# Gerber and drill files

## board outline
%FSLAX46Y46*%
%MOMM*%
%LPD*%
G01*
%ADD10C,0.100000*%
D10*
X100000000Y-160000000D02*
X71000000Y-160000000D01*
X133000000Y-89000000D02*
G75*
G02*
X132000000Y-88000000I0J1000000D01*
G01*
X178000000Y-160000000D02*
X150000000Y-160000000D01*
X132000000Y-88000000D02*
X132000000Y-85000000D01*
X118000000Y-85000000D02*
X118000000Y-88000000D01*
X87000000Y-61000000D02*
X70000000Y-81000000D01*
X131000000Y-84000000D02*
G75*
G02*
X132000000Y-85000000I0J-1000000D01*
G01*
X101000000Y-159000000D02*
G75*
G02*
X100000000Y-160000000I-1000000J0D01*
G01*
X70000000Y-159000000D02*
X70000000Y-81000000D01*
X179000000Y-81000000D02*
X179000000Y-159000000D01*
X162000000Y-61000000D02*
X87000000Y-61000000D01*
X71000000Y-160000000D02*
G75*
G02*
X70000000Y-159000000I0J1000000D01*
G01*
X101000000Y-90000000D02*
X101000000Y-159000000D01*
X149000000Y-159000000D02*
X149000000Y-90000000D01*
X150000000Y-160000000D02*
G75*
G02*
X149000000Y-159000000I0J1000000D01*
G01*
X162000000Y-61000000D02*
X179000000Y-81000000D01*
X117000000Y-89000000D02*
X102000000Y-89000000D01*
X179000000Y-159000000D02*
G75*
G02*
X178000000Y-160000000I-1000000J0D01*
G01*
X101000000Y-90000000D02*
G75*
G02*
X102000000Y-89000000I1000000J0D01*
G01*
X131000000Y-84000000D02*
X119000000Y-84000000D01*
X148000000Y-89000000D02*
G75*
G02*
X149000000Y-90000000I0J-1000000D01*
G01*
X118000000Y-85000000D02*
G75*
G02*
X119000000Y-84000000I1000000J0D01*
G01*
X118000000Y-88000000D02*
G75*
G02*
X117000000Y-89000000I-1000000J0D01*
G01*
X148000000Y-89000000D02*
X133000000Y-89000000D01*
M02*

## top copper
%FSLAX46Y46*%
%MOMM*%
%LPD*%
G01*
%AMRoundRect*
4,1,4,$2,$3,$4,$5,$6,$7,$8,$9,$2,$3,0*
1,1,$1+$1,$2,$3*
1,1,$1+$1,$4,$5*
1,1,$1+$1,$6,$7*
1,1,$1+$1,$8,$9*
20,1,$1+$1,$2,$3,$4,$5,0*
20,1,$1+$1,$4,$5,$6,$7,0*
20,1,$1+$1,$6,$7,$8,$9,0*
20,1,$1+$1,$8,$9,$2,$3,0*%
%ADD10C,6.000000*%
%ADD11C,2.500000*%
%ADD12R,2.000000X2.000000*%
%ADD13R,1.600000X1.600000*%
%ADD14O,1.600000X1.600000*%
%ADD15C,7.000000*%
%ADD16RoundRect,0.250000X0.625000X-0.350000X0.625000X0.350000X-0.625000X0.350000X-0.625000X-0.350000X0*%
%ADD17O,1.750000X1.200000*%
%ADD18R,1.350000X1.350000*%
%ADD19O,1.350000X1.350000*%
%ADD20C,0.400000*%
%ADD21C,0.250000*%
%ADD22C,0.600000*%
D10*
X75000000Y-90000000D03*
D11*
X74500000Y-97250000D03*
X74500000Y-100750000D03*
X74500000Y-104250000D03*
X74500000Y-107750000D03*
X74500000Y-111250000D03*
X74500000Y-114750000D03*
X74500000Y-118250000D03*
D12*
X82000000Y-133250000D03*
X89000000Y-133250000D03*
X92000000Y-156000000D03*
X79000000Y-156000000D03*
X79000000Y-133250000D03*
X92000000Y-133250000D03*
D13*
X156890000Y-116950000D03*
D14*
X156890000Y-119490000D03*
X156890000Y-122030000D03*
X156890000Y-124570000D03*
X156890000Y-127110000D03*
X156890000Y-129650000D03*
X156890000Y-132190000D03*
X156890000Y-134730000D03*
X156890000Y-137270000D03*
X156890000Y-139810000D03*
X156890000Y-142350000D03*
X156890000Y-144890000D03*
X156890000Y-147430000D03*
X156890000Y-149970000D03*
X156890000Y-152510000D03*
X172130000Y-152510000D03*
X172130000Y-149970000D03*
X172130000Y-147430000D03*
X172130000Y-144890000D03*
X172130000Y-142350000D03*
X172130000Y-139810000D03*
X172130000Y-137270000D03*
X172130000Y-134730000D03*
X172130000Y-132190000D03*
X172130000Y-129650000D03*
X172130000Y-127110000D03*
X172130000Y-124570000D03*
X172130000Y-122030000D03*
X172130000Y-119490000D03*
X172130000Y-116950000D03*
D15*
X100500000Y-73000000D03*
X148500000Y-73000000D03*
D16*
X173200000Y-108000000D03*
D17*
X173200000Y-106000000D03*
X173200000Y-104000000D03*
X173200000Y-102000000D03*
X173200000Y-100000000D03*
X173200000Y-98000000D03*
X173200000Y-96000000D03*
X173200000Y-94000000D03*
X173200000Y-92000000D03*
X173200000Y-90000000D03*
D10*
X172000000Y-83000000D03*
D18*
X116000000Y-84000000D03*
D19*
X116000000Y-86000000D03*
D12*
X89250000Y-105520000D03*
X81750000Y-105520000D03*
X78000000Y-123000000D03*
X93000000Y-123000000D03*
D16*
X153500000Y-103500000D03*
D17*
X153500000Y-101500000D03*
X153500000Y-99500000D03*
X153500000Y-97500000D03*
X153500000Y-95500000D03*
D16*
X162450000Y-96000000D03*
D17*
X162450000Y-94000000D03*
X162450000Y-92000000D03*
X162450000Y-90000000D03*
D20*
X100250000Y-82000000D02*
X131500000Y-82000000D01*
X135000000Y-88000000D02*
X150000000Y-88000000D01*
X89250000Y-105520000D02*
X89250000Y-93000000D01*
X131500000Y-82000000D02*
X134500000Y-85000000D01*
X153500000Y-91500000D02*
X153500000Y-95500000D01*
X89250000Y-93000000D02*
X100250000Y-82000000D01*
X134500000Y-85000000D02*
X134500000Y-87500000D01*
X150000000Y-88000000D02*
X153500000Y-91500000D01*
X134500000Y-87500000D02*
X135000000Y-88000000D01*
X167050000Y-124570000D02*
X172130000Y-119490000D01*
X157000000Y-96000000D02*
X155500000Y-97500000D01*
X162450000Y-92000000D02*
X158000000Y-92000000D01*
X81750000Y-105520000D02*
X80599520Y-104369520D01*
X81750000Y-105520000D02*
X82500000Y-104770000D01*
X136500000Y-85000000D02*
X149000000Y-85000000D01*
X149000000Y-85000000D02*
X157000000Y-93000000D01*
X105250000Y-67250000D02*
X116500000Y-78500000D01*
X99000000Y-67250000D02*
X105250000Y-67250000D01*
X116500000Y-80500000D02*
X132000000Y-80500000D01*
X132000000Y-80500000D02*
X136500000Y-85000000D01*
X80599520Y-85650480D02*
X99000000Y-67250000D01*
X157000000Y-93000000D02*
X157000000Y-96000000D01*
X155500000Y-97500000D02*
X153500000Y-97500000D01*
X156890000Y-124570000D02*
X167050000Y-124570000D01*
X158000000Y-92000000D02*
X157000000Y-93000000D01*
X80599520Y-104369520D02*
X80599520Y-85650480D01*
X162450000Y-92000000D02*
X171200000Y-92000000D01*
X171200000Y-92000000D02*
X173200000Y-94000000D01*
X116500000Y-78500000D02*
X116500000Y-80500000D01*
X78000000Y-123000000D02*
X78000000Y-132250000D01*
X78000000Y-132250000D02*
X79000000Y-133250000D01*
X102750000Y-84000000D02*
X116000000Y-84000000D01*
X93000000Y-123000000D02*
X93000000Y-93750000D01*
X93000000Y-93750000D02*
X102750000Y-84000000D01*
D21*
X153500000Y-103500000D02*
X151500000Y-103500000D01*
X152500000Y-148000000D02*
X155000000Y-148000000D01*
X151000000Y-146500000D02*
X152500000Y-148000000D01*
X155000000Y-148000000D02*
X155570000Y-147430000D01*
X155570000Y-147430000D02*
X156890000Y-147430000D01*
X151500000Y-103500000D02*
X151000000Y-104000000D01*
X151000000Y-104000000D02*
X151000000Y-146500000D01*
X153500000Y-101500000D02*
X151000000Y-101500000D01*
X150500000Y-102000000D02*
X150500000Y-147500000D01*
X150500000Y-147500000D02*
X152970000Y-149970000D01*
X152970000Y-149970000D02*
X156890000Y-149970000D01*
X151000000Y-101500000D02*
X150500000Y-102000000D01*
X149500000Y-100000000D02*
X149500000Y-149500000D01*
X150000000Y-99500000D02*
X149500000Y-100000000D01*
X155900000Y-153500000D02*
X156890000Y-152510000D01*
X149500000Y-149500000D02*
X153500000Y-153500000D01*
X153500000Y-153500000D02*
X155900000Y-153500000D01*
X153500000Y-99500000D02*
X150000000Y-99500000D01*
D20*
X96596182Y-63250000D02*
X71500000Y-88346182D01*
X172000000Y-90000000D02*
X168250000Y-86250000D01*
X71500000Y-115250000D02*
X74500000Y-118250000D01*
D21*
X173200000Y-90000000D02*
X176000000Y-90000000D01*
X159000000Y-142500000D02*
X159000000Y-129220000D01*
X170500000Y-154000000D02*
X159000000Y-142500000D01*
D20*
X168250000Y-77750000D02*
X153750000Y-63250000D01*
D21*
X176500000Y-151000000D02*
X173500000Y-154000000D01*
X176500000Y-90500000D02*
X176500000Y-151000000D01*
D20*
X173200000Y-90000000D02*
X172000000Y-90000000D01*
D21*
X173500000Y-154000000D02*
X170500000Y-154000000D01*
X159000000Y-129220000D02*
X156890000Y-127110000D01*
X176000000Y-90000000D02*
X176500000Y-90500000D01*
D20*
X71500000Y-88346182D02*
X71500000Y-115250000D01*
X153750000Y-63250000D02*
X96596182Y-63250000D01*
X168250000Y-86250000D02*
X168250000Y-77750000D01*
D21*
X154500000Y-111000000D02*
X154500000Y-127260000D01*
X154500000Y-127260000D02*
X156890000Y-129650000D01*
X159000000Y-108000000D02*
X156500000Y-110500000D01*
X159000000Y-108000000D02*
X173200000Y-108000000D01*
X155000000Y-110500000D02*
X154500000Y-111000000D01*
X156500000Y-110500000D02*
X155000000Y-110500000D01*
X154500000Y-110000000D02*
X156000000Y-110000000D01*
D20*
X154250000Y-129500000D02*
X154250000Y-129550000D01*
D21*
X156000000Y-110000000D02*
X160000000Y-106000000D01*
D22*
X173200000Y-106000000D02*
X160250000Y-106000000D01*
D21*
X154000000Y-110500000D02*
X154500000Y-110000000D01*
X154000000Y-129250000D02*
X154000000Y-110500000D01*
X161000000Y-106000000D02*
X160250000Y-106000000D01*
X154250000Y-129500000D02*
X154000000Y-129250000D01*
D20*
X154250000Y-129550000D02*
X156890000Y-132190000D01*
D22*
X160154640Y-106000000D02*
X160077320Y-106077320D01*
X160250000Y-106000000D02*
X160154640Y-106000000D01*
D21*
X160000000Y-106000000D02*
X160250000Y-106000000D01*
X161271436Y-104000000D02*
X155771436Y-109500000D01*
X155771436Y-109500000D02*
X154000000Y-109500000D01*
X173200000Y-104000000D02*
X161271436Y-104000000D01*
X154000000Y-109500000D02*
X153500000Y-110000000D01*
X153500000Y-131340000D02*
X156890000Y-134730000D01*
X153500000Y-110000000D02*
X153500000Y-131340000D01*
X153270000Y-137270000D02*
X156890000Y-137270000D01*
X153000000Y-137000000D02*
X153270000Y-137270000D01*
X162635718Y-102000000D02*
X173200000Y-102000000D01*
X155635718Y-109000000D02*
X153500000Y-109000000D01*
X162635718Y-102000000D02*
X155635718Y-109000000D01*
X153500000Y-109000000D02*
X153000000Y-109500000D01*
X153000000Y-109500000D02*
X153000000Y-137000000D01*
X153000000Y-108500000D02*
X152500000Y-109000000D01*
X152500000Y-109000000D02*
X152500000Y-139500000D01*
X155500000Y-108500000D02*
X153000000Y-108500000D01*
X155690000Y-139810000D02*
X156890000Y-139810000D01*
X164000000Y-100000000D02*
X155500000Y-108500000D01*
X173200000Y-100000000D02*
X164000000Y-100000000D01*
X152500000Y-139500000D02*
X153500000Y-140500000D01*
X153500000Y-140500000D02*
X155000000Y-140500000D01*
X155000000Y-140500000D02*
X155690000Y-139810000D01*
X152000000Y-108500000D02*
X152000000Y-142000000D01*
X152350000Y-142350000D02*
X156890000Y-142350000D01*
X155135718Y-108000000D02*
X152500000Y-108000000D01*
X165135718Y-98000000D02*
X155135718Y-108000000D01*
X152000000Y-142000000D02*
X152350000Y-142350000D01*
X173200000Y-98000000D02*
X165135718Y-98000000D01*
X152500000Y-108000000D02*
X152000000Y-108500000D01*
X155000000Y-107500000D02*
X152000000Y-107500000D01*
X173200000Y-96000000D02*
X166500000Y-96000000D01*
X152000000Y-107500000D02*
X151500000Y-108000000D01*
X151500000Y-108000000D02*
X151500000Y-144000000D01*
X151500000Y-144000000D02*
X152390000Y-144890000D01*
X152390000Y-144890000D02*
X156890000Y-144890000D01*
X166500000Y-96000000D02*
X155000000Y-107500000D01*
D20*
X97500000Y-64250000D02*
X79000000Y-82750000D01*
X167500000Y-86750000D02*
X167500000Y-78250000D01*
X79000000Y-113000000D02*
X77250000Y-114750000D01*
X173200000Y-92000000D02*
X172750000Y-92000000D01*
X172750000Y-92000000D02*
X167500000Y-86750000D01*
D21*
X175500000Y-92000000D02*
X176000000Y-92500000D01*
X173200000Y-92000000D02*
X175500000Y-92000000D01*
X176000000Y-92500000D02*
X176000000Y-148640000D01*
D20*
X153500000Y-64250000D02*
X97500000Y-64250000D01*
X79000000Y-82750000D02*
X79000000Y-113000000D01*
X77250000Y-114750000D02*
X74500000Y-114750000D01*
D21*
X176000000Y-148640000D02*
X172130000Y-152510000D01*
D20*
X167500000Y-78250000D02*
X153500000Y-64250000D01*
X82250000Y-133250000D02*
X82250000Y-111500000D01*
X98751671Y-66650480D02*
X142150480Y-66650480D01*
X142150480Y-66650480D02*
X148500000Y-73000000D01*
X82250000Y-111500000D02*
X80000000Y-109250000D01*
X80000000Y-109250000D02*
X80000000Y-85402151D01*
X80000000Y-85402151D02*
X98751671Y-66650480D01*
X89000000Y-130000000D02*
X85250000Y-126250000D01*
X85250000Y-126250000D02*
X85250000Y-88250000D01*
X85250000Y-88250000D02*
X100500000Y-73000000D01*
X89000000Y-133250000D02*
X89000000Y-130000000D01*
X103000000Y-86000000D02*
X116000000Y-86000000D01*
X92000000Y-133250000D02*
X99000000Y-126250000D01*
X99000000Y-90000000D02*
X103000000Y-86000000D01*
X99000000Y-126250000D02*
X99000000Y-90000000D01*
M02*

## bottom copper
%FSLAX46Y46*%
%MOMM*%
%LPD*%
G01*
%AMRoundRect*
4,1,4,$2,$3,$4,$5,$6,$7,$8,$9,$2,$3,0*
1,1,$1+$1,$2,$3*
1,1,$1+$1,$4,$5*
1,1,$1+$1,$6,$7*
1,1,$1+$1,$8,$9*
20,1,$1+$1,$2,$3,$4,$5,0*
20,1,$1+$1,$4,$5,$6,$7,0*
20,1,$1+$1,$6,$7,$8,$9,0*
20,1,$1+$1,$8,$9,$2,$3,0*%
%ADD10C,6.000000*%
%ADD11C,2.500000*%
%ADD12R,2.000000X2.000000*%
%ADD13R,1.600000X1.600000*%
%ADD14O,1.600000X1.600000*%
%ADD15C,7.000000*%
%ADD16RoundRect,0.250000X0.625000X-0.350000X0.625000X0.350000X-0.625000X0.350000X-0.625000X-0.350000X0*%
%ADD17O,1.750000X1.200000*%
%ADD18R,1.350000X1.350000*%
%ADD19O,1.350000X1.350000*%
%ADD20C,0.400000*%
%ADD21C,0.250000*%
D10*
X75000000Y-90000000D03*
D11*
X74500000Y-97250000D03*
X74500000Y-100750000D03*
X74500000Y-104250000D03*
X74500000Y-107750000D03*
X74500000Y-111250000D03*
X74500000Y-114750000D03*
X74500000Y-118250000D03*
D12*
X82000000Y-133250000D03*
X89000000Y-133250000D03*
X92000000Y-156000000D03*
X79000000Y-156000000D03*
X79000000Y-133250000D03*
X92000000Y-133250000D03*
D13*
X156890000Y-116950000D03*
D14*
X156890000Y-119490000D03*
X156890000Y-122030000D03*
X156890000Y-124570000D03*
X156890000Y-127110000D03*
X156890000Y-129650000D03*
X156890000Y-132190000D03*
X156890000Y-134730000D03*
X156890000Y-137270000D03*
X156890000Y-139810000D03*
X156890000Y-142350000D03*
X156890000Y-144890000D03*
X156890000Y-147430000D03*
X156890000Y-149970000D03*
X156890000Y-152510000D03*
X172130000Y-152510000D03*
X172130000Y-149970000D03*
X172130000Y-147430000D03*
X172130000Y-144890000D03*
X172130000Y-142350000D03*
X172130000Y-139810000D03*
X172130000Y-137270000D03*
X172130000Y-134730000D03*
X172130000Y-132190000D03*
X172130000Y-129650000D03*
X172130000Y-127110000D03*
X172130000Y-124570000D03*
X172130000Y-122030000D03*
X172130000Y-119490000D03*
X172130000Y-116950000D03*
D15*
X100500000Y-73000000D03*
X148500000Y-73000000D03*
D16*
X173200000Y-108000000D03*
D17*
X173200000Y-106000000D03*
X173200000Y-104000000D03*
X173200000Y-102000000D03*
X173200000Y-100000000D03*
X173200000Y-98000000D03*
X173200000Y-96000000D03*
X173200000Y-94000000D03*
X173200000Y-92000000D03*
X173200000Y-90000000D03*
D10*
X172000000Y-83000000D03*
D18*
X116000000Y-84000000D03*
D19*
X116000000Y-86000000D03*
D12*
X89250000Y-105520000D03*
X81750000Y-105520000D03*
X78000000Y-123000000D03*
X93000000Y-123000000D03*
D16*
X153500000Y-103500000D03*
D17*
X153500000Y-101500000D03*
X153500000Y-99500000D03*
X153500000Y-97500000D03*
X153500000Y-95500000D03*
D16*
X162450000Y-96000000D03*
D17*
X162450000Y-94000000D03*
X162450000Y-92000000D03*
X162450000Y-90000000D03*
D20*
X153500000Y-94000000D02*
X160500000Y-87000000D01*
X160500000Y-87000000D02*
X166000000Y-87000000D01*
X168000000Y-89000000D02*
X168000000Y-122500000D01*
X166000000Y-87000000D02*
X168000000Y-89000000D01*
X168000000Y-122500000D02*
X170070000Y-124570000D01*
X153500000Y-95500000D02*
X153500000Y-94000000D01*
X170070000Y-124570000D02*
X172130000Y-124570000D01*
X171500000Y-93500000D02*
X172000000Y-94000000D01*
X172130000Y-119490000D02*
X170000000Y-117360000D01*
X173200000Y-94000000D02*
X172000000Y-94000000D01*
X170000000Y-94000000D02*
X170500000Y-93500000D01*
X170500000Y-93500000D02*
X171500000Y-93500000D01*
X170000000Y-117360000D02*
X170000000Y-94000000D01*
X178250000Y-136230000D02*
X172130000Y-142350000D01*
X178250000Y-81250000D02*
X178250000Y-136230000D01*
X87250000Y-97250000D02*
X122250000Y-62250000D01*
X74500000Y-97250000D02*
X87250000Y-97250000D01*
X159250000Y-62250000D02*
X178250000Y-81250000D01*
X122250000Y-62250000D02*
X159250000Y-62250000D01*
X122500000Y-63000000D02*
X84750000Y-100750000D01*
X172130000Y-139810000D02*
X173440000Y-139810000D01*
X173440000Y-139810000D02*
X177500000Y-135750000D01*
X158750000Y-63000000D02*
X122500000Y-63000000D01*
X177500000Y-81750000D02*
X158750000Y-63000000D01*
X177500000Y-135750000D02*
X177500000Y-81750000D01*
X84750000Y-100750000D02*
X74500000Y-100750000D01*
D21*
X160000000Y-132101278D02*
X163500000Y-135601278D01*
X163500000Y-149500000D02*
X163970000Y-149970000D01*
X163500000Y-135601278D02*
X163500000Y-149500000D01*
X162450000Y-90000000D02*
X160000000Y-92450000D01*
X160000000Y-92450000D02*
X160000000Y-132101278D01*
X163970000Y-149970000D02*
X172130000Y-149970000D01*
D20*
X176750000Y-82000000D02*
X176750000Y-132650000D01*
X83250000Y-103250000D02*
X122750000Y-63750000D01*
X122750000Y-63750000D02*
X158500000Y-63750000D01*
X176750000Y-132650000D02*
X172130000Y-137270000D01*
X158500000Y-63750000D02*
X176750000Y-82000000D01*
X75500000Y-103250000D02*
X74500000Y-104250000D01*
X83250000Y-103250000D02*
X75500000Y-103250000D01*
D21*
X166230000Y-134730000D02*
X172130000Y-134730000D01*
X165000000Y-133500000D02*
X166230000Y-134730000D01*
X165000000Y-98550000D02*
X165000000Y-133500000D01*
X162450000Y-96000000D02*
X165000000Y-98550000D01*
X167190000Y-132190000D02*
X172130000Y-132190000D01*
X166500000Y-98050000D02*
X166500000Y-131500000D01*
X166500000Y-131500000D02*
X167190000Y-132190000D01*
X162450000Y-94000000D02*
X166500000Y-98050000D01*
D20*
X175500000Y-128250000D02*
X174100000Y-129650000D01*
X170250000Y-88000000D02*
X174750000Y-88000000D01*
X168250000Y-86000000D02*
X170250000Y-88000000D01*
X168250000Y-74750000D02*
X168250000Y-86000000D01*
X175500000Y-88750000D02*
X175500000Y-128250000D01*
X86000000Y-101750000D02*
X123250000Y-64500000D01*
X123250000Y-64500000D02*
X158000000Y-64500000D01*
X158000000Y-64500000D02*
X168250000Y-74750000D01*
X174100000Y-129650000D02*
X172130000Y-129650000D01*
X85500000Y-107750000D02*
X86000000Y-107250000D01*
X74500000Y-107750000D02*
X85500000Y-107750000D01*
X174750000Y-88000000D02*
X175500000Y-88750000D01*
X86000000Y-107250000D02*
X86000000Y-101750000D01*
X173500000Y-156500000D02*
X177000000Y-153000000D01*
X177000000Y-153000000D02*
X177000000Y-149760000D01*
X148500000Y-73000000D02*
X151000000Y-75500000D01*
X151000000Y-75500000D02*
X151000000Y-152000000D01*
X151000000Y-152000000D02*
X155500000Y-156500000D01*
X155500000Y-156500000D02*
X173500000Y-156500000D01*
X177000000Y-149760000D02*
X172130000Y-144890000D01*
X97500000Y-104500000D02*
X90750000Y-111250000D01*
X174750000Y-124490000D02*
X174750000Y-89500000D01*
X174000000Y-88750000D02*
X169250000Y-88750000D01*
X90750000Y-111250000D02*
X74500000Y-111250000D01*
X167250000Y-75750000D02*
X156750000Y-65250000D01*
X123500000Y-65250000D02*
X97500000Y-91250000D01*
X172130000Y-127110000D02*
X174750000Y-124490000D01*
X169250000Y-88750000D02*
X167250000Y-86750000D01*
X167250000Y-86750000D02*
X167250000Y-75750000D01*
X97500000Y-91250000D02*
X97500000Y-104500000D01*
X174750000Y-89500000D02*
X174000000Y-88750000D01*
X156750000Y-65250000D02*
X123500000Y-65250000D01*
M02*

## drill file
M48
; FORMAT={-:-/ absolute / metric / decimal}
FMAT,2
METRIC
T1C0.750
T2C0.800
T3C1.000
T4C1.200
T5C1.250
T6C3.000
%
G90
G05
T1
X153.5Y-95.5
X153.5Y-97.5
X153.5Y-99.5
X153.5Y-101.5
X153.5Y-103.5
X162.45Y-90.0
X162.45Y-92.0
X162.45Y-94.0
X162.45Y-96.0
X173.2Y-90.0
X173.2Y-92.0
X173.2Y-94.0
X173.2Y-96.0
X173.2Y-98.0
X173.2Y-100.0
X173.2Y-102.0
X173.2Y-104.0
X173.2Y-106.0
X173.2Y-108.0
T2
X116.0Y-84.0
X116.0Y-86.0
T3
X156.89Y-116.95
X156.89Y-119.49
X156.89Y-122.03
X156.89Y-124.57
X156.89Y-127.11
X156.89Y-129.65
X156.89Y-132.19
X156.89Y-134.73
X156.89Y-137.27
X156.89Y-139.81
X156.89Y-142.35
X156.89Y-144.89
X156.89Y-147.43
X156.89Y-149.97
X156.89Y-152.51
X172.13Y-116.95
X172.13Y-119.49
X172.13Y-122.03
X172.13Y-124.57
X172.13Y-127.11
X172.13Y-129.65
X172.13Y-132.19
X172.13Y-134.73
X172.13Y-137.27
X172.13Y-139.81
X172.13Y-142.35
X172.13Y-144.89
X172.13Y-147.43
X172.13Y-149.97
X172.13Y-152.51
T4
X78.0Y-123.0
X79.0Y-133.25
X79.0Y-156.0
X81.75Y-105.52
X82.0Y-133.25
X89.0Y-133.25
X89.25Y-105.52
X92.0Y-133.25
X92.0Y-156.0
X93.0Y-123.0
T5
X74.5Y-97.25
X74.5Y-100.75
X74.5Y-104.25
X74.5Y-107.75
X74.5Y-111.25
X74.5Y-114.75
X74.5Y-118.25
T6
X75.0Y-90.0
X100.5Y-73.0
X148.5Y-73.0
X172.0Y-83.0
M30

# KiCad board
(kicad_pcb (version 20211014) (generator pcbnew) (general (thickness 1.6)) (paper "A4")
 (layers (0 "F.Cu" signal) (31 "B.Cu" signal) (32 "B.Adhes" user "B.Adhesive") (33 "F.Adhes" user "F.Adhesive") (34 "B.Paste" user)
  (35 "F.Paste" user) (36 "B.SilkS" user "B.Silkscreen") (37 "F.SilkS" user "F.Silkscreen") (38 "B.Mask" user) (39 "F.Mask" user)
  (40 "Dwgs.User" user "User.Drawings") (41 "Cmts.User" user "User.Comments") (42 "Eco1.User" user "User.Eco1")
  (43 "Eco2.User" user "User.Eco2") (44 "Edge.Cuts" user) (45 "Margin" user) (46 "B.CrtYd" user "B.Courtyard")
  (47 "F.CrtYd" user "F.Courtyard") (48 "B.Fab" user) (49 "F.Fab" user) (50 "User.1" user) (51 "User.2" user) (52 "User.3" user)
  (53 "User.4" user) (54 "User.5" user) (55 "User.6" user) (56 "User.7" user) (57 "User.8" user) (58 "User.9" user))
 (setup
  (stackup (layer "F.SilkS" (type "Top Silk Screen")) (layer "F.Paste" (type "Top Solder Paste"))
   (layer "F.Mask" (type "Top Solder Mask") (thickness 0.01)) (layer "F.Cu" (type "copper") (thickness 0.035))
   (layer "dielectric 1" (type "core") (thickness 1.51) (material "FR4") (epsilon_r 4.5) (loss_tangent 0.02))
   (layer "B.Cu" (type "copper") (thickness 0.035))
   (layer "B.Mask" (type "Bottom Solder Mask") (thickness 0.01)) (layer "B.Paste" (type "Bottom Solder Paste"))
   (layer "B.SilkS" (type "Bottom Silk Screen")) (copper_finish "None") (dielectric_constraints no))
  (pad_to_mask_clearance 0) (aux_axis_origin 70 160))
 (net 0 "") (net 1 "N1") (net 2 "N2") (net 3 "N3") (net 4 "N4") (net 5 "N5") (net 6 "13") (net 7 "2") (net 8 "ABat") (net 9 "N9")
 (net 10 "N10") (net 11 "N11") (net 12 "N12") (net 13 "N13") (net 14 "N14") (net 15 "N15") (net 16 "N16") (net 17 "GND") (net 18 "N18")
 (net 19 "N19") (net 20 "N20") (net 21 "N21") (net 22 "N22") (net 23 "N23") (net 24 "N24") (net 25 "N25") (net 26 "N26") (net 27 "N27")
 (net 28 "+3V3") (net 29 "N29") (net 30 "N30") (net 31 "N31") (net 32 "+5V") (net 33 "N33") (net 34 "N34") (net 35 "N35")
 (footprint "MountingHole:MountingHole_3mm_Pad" (layer "F.Cu") (at 75 90)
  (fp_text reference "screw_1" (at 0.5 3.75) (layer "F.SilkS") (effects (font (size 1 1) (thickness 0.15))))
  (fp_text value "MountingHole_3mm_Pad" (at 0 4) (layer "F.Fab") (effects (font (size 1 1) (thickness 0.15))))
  (pad "1" thru_hole circle (at 0 0) (size 6 6) (drill 3) (layers *.Cu *.Mask)))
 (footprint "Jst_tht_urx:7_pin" (layer "F.Cu") (at 74.5 97.25)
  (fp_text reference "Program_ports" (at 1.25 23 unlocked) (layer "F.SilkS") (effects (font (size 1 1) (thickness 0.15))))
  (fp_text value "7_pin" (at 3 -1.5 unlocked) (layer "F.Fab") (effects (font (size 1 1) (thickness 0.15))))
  (pad "1" thru_hole circle (at 0 0) (size 2.5 2.5) (drill 1.25) (layers *.Cu *.Mask) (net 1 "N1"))
  (pad "2" thru_hole circle (at 0 3.5) (size 2.5 2.5) (drill 1.25) (layers *.Cu *.Mask) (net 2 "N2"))
  (pad "3" thru_hole circle (at 0 7) (size 2.5 2.5) (drill 1.25) (layers *.Cu *.Mask) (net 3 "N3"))
  (pad "4" thru_hole circle (at 0 10.5) (size 2.5 2.5) (drill 1.25) (layers *.Cu *.Mask) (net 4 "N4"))
  (pad "5" thru_hole circle (at 0 14) (size 2.5 2.5) (drill 1.25) (layers *.Cu *.Mask) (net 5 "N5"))
  (pad "6" thru_hole circle (at 0 17.5) (size 2.5 2.5) (drill 1.25) (layers *.Cu *.Mask) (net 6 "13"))
  (pad "7" thru_hole circle (at 0 21) (size 2.5 2.5) (drill 1.25) (layers *.Cu *.Mask) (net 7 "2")))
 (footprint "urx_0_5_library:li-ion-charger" (layer "F.Cu") (at 85.5 145 -90)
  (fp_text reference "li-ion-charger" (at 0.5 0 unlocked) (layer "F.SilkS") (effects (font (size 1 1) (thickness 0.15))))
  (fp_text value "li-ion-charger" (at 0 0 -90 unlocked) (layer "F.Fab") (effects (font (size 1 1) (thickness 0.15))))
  (pad "1" thru_hole rect (at -11.75 3.5 270) (size 2 2) (drill 1.2) (layers *.Cu *.Mask) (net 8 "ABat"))
  (pad "2" thru_hole rect (at -11.75 -3.5 270) (size 2 2) (drill 1.2) (layers *.Cu *.Mask) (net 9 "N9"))
  (pad "3" thru_hole rect (at 11 -6.5 270) (size 2 2) (drill 1.2) (layers *.Cu *.Mask) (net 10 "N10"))
  (pad "4" thru_hole rect (at 11 6.5 270) (size 2 2) (drill 1.2) (layers *.Cu *.Mask) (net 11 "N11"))
  (pad "5" thru_hole rect (at -11.75 6.5 270) (size 2 2) (drill 1.2) (layers *.Cu *.Mask) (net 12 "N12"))
  (pad "6" thru_hole rect (at -11.75 -6.5 270) (size 2 2) (drill 1.2) (layers *.Cu *.Mask) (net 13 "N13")))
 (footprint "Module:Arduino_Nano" (layer "F.Cu") (at 156.89 116.95)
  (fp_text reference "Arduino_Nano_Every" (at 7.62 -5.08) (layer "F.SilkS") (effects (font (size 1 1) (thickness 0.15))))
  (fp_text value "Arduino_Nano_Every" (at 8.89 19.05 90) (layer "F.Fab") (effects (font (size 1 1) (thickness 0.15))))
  (pad "1" thru_hole rect (at 0 0) (size 1.6 1.6) (drill 1) (layers *.Cu *.Mask) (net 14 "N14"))
  (pad "2" thru_hole oval (at 0 2.54) (size 1.6 1.6) (drill 1) (layers *.Cu *.Mask) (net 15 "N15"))
  (pad "3" thru_hole oval (at 0 5.08) (size 1.6 1.6) (drill 1) (layers *.Cu *.Mask) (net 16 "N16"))
  (pad "4" thru_hole oval (at 0 7.62) (size 1.6 1.6) (drill 1) (layers *.Cu *.Mask) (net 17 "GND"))
  (pad "5" thru_hole oval (at 0 10.16) (size 1.6 1.6) (drill 1) (layers *.Cu *.Mask) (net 7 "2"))
  (pad "6" thru_hole oval (at 0 12.7) (size 1.6 1.6) (drill 1) (layers *.Cu *.Mask) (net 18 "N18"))
  (pad "7" thru_hole oval (at 0 15.24) (size 1.6 1.6) (drill 1) (layers *.Cu *.Mask) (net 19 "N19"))
  (pad "8" thru_hole oval (at 0 17.78) (size 1.6 1.6) (drill 1) (layers *.Cu *.Mask) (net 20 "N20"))
  (pad "9" thru_hole oval (at 0 20.32) (size 1.6 1.6) (drill 1) (layers *.Cu *.Mask) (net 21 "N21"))
  (pad "10" thru_hole oval (at 0 22.86) (size 1.6 1.6) (drill 1) (layers *.Cu *.Mask) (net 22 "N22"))
  (pad "11" thru_hole oval (at 0 25.4) (size 1.6 1.6) (drill 1) (layers *.Cu *.Mask) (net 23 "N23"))
  (pad "12" thru_hole oval (at 0 27.94) (size 1.6 1.6) (drill 1) (layers *.Cu *.Mask) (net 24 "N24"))
  (pad "13" thru_hole oval (at 0 30.48) (size 1.6 1.6) (drill 1) (layers *.Cu *.Mask) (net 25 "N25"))
  (pad "14" thru_hole oval (at 0 33.02) (size 1.6 1.6) (drill 1) (layers *.Cu *.Mask) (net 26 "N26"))
  (pad "15" thru_hole oval (at 0 35.56) (size 1.6 1.6) (drill 1) (layers *.Cu *.Mask) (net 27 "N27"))
  (pad "16" thru_hole oval (at 15.24 35.56) (size 1.6 1.6) (drill 1) (layers *.Cu *.Mask) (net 6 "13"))
  (pad "17" thru_hole oval (at 15.24 33.02) (size 1.6 1.6) (drill 1) (layers *.Cu *.Mask) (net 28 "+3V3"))
  (pad "18" thru_hole oval (at 15.24 30.48) (size 1.6 1.6) (drill 1) (layers *.Cu *.Mask) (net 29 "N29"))
  (pad "19" thru_hole oval (at 15.24 27.94) (size 1.6 1.6) (drill 1) (layers *.Cu *.Mask) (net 8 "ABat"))
  (pad "20" thru_hole oval (at 15.24 25.4) (size 1.6 1.6) (drill 1) (layers *.Cu *.Mask) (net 1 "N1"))
  (pad "21" thru_hole oval (at 15.24 22.86) (size 1.6 1.6) (drill 1) (layers *.Cu *.Mask) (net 2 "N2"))
  (pad "22" thru_hole oval (at 15.24 20.32) (size 1.6 1.6) (drill 1) (layers *.Cu *.Mask) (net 3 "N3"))
  (pad "23" thru_hole oval (at 15.24 17.78) (size 1.6 1.6) (drill 1) (layers *.Cu *.Mask) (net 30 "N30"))
  (pad "24" thru_hole oval (at 15.24 15.24) (size 1.6 1.6) (drill 1) (layers *.Cu *.Mask) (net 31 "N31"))
  (pad "25" thru_hole oval (at 15.24 12.7) (size 1.6 1.6) (drill 1) (layers *.Cu *.Mask) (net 4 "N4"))
  (pad "26" thru_hole oval (at 15.24 10.16) (size 1.6 1.6) (drill 1) (layers *.Cu *.Mask) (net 5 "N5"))
  (pad "27" thru_hole oval (at 15.24 7.62) (size 1.6 1.6) (drill 1) (layers *.Cu *.Mask) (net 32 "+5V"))
  (pad "28" thru_hole oval (at 15.24 5.08) (size 1.6 1.6) (drill 1) (layers *.Cu *.Mask) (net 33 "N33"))
  (pad "29" thru_hole oval (at 15.24 2.54) (size 1.6 1.6) (drill 1) (layers *.Cu *.Mask) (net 17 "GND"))
  (pad "30" thru_hole oval (at 15.24 0) (size 1.6 1.6) (drill 1) (layers *.Cu *.Mask) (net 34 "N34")))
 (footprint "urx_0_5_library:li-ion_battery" (layer "F.Cu") (at 124.5 73 90)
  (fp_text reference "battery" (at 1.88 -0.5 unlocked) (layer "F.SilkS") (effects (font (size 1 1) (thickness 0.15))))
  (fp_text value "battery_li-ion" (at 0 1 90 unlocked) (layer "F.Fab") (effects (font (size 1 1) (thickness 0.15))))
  (pad "1" thru_hole circle (at 0 -24 90) (size 7 7) (drill 3) (layers *.Cu *.Mask) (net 9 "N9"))
  (pad "2" thru_hole circle (at 0 24 90) (size 7 7) (drill 3) (layers *.Cu *.Mask) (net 8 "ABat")))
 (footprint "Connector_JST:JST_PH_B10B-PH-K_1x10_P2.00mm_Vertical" (layer "F.Cu") (at 173.2 108 90)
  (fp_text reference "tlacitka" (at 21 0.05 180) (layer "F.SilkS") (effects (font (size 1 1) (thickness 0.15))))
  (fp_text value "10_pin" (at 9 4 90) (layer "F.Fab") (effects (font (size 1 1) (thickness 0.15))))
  (pad "1" thru_hole roundrect (at 0 0 90) (size 1.2 1.75) (drill 0.75) (layers *.Cu *.Mask) (roundrect_rratio 0.2083333333) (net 18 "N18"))
  (pad "2" thru_hole oval (at 2 0 90) (size 1.2 1.75) (drill 0.75) (layers *.Cu *.Mask) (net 19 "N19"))
  (pad "3" thru_hole oval (at 4 0 90) (size 1.2 1.75) (drill 0.75) (layers *.Cu *.Mask) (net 20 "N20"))
  (pad "4" thru_hole oval (at 6 0 90) (size 1.2 1.75) (drill 0.75) (layers *.Cu *.Mask) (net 21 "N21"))
  (pad "5" thru_hole oval (at 8 0 90) (size 1.2 1.75) (drill 0.75) (layers *.Cu *.Mask) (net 22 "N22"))
  (pad "6" thru_hole oval (at 10 0 90) (size 1.2 1.75) (drill 0.75) (layers *.Cu *.Mask) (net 23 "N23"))
  (pad "7" thru_hole oval (at 12 0 90) (size 1.2 1.75) (drill 0.75) (layers *.Cu *.Mask) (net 24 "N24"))
  (pad "8" thru_hole oval (at 14 0 90) (size 1.2 1.75) (drill 0.75) (layers *.Cu *.Mask) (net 17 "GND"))
  (pad "9" thru_hole oval (at 16 0 90) (size 1.2 1.75) (drill 0.75) (layers *.Cu *.Mask) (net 6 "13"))
  (pad "10" thru_hole oval (at 18 0 90) (size 1.2 1.75) (drill 0.75) (layers *.Cu *.Mask) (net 7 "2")))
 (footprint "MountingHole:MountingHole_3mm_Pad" (layer "F.Cu") (at 172 83)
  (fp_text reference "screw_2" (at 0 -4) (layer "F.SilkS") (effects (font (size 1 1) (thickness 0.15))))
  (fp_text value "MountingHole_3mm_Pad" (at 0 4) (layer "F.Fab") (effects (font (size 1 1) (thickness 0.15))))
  (pad "1" thru_hole circle (at 0 0) (size 6 6) (drill 3) (layers *.Cu *.Mask)))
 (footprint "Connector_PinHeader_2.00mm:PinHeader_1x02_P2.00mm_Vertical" (layer "F.Cu") (at 116 84)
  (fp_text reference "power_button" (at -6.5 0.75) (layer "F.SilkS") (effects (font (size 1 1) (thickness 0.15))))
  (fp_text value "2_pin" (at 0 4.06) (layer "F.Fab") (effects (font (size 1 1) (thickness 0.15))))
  (pad "1" thru_hole rect (at 0 0) (size 1.35 1.35) (drill 0.8) (layers *.Cu *.Mask) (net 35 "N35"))
  (pad "2" thru_hole oval (at 0 2) (size 1.35 1.35) (drill 0.8) (layers *.Cu *.Mask) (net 13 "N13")))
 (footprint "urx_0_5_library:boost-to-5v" (layer "F.Cu") (at 85.5 115 -90)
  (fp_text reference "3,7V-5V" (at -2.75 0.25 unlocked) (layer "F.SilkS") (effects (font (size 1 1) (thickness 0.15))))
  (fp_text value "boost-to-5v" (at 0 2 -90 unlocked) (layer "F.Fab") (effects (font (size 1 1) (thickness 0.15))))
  (pad "1" thru_hole rect (at -9.48 -3.75 270) (size 2 2) (drill 1.2) (layers *.Cu *.Mask) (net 32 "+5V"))
  (pad "2" thru_hole rect (at -9.48 3.75 270) (size 2 2) (drill 1.2) (layers *.Cu *.Mask) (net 17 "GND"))
  (pad "3" thru_hole rect (at 8 7.5 270) (size 2 2) (drill 1.2) (layers *.Cu *.Mask) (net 12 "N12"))
  (pad "4" thru_hole rect (at 8 -7.5 270) (size 2 2) (drill 1.2) (layers *.Cu *.Mask) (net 35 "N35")))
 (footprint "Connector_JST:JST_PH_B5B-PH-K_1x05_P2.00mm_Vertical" (layer "F.Cu") (at 153.5 103.5 90)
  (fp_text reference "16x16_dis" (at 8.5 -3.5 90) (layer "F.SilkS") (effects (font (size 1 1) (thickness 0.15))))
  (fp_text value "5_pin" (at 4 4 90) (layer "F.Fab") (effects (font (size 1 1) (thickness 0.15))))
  (pad "1" thru_hole roundrect (at 0 0 90) (size 1.2 1.75) (drill 0.75) (layers *.Cu *.Mask) (roundrect_rratio 0.2083333333) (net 25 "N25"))
  (pad "2" thru_hole oval (at 2 0 90) (size 1.2 1.75) (drill 0.75) (layers *.Cu *.Mask) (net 26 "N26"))
  (pad "3" thru_hole oval (at 4 0 90) (size 1.2 1.75) (drill 0.75) (layers *.Cu *.Mask) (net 27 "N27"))
  (pad "4" thru_hole oval (at 6 0 90) (size 1.2 1.75) (drill 0.75) (layers *.Cu *.Mask) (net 17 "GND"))
  (pad "5" thru_hole oval (at 8 0 90) (size 1.2 1.75) (drill 0.75) (layers *.Cu *.Mask) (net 32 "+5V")))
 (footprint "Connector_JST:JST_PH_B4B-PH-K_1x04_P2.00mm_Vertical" (layer "F.Cu") (at 162.45 96 90)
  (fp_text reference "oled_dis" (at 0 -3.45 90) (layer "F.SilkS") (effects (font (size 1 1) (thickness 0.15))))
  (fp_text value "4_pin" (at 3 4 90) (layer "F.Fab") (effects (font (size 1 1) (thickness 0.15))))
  (pad "1" thru_hole roundrect (at 0 0 90) (size 1.2 1.75) (drill 0.75) (layers *.Cu *.Mask) (roundrect_rratio 0.2083333333) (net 30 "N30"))
  (pad "2" thru_hole oval (at 2 0 90) (size 1.2 1.75) (drill 0.75) (layers *.Cu *.Mask) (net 31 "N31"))
  (pad "3" thru_hole oval (at 4 0 90) (size 1.2 1.75) (drill 0.75) (layers *.Cu *.Mask) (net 17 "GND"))
  (pad "4" thru_hole oval (at 6 0 90) (size 1.2 1.75) (drill 0.75) (layers *.Cu *.Mask) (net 28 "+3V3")))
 (gr_line (start 100 160) (end 71 160) (layer "Edge.Cuts") (width 0.1))
 (gr_arc (start 133 89) (mid 132.292893 88.707107) (end 132 88) (layer "Edge.Cuts") (width 0.1))
 (gr_line (start 178 160) (end 150 160) (layer "Edge.Cuts") (width 0.1))
 (gr_line (start 132 88) (end 132 85) (layer "Edge.Cuts") (width 0.1))
 (gr_line (start 118 85) (end 118 88) (layer "Edge.Cuts") (width 0.1))
 (gr_line (start 87 61) (end 70 81) (layer "Edge.Cuts") (width 0.1))
 (gr_arc (start 131 84) (mid 131.707107 84.292893) (end 132 85) (layer "Edge.Cuts") (width 0.1))
 (gr_arc (start 101 159) (mid 100.707107 159.707107) (end 100 160) (layer "Edge.Cuts") (width 0.1))
 (gr_line (start 70 159) (end 70 81) (layer "Edge.Cuts") (width 0.1))
 (gr_line (start 179 81) (end 179 159) (layer "Edge.Cuts") (width 0.1))
 (gr_line (start 162 61) (end 87 61) (layer "Edge.Cuts") (width 0.1))
 (gr_arc (start 71 160) (mid 70.292893 159.707107) (end 70 159) (layer "Edge.Cuts") (width 0.1))
 (gr_line (start 101 90) (end 101 159) (layer "Edge.Cuts") (width 0.1))
 (gr_line (start 149 159) (end 149 90) (layer "Edge.Cuts") (width 0.1))
 (gr_arc (start 150 160) (mid 149.292893 159.707107) (end 149 159) (layer "Edge.Cuts") (width 0.1))
 (gr_line (start 162 61) (end 179 81) (layer "Edge.Cuts") (width 0.1))
 (gr_line (start 117 89) (end 102 89) (layer "Edge.Cuts") (width 0.1))
 (gr_arc (start 179 159) (mid 178.707107 159.707107) (end 178 160) (layer "Edge.Cuts") (width 0.1))
 (gr_arc (start 101 90) (mid 101.292893 89.292893) (end 102 89) (layer "Edge.Cuts") (width 0.1))
 (gr_line (start 131 84) (end 119 84) (layer "Edge.Cuts") (width 0.1))
 (gr_arc (start 148 89) (mid 148.707107 89.292893) (end 149 90) (layer "Edge.Cuts") (width 0.1))
 (gr_arc (start 118 85) (mid 118.292893 84.292893) (end 119 84) (layer "Edge.Cuts") (width 0.1))
 (gr_arc (start 118 88) (mid 117.707107 88.707107) (end 117 89) (layer "Edge.Cuts") (width 0.1))
 (gr_line (start 148 89) (end 133 89) (layer "Edge.Cuts") (width 0.1))
 (segment (start 100.25 82) (end 131.5 82) (width 0.4) (layer "F.Cu") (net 32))
 (segment (start 135 88) (end 150 88) (width 0.4) (layer "F.Cu") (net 32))
 (segment (start 89.25 105.52) (end 89.25 93) (width 0.4) (layer "F.Cu") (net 32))
 (segment (start 131.5 82) (end 134.5 85) (width 0.4) (layer "F.Cu") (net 32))
 (segment (start 153.5 91.5) (end 153.5 95.5) (width 0.4) (layer "F.Cu") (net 32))
 (segment (start 89.25 93) (end 100.25 82) (width 0.4) (layer "F.Cu") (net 32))
 (segment (start 134.5 85) (end 134.5 87.5) (width 0.4) (layer "F.Cu") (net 32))
 (segment (start 150 88) (end 153.5 91.5) (width 0.4) (layer "F.Cu") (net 32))
 (segment (start 134.5 87.5) (end 135 88) (width 0.4) (layer "F.Cu") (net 32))
 (segment (start 153.5 94) (end 160.5 87) (width 0.4) (layer "B.Cu") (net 32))
 (segment (start 160.5 87) (end 166 87) (width 0.4) (layer "B.Cu") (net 32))
 (segment (start 168 89) (end 168 122.5) (width 0.4) (layer "B.Cu") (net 32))
 (segment (start 166 87) (end 168 89) (width 0.4) (layer "B.Cu") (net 32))
 (segment (start 168 122.5) (end 170.07 124.57) (width 0.4) (layer "B.Cu") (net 32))
 (segment (start 153.5 95.5) (end 153.5 94) (width 0.4) (layer "B.Cu") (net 32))
 (segment (start 170.07 124.57) (end 172.13 124.57) (width 0.4) (layer "B.Cu") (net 32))
 (segment (start 167.05 124.57) (end 172.13 119.49) (width 0.4) (layer "F.Cu") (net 17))
 (segment (start 157 96) (end 155.5 97.5) (width 0.4) (layer "F.Cu") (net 17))
 (segment (start 162.45 92) (end 158 92) (width 0.4) (layer "F.Cu") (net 17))
 (segment (start 81.75 105.52) (end 80.59952 104.36952) (width 0.4) (layer "F.Cu") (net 17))
 (segment (start 81.75 105.52) (end 82.5 104.77) (width 0.4) (layer "F.Cu") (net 17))
 (segment (start 136.5 85) (end 149 85) (width 0.4) (layer "F.Cu") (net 17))
 (segment (start 149 85) (end 157 93) (width 0.4) (layer "F.Cu") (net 17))
 (segment (start 105.25 67.25) (end 116.5 78.5) (width 0.4) (layer "F.Cu") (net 17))
 (segment (start 99 67.25) (end 105.25 67.25) (width 0.4) (layer "F.Cu") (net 17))
 (segment (start 116.5 80.5) (end 132 80.5) (width 0.4) (layer "F.Cu") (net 17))
 (segment (start 132 80.5) (end 136.5 85) (width 0.4) (layer "F.Cu") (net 17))
 (segment (start 80.59952 85.65048) (end 99 67.25) (width 0.4) (layer "F.Cu") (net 17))
 (segment (start 157 93) (end 157 96) (width 0.4) (layer "F.Cu") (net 17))
 (segment (start 155.5 97.5) (end 153.5 97.5) (width 0.4) (layer "F.Cu") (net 17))
 (segment (start 156.89 124.57) (end 167.05 124.57) (width 0.4) (layer "F.Cu") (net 17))
 (segment (start 158 92) (end 157 93) (width 0.4) (layer "F.Cu") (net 17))
 (segment (start 80.59952 104.36952) (end 80.59952 85.65048) (width 0.4) (layer "F.Cu") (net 17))
 (segment (start 162.45 92) (end 171.2 92) (width 0.4) (layer "F.Cu") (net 17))
 (segment (start 171.2 92) (end 173.2 94) (width 0.4) (layer "F.Cu") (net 17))
 (segment (start 116.5 78.5) (end 116.5 80.5) (width 0.4) (layer "F.Cu") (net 17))
 (segment (start 171.5 93.5) (end 172 94) (width 0.4) (layer "B.Cu") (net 17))
 (segment (start 172.13 119.49) (end 170 117.36) (width 0.4) (layer "B.Cu") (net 17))
 (segment (start 173.2 94) (end 172 94) (width 0.4) (layer "B.Cu") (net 17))
 (segment (start 170 94) (end 170.5 93.5) (width 0.4) (layer "B.Cu") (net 17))
 (segment (start 170.5 93.5) (end 171.5 93.5) (width 0.4) (layer "B.Cu") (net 17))
 (segment (start 170 117.36) (end 170 94) (width 0.4) (layer "B.Cu") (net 17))
 (segment (start 78 123) (end 78 132.25) (width 0.4) (layer "F.Cu") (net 12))
 (segment (start 78 132.25) (end 79 133.25) (width 0.4) (layer "F.Cu") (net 12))
 (segment (start 102.75 84) (end 116 84) (width 0.4) (layer "F.Cu") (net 35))
 (segment (start 93 123) (end 93 93.75) (width 0.4) (layer "F.Cu") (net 35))
 (segment (start 93 93.75) (end 102.75 84) (width 0.4) (layer "F.Cu") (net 35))
 (segment (start 153.5 103.5) (end 151.5 103.5) (width 0.25) (layer "F.Cu") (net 25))
 (segment (start 152.5 148) (end 155 148) (width 0.25) (layer "F.Cu") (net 25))
 (segment (start 151 146.5) (end 152.5 148) (width 0.25) (layer "F.Cu") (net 25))
 (segment (start 155 148) (end 155.57 147.43) (width 0.25) (layer "F.Cu") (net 25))
 (segment (start 155.57 147.43) (end 156.89 147.43) (width 0.25) (layer "F.Cu") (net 25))
 (segment (start 151.5 103.5) (end 151 104) (width 0.25) (layer "F.Cu") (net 25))
 (segment (start 151 104) (end 151 146.5) (width 0.25) (layer "F.Cu") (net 25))
 (segment (start 153.5 101.5) (end 151 101.5) (width 0.25) (layer "F.Cu") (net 26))
 (segment (start 150.5 102) (end 150.5 147.5) (width 0.25) (layer "F.Cu") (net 26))
 (segment (start 150.5 147.5) (end 152.97 149.97) (width 0.25) (layer "F.Cu") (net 26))
 (segment (start 152.97 149.97) (end 156.89 149.97) (width 0.25) (layer "F.Cu") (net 26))
 (segment (start 151 101.5) (end 150.5 102) (width 0.25) (layer "F.Cu") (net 26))
 (segment (start 149.5 100) (end 149.5 149.5) (width 0.25) (layer "F.Cu") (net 27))
 (segment (start 150 99.5) (end 149.5 100) (width 0.25) (layer "F.Cu") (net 27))
 (segment (start 155.9 153.5) (end 156.89 152.51) (width 0.25) (layer "F.Cu") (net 27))
 (segment (start 149.5 149.5) (end 153.5 153.5) (width 0.25) (layer "F.Cu") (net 27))
 (segment (start 153.5 153.5) (end 155.9 153.5) (width 0.25) (layer "F.Cu") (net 27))
 (segment (start 153.5 99.5) (end 150 99.5) (width 0.25) (layer "F.Cu") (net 27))
 (segment (start 96.596182 63.25) (end 71.5 88.346182) (width 0.4) (layer "F.Cu") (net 7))
 (segment (start 172 90) (end 168.25 86.25) (width 0.4) (layer "F.Cu") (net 7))
 (segment (start 71.5 115.25) (end 74.5 118.25) (width 0.4) (layer "F.Cu") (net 7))
 (segment (start 173.2 90) (end 176 90) (width 0.25) (layer "F.Cu") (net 7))
 (segment (start 159 142.5) (end 159 129.22) (width 0.25) (layer "F.Cu") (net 7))
 (segment (start 170.5 154) (end 159 142.5) (width 0.25) (layer "F.Cu") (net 7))
 (segment (start 168.25 77.75) (end 153.75 63.25) (width 0.4) (layer "F.Cu") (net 7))
 (segment (start 176.5 151) (end 173.5 154) (width 0.25) (layer "F.Cu") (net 7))
 (segment (start 176.5 90.5) (end 176.5 151) (width 0.25) (layer "F.Cu") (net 7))
 (segment (start 173.2 90) (end 172 90) (width 0.4) (layer "F.Cu") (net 7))
 (segment (start 173.5 154) (end 170.5 154) (width 0.25) (layer "F.Cu") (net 7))
 (segment (start 159 129.22) (end 156.89 127.11) (width 0.25) (layer "F.Cu") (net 7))
 (segment (start 176 90) (end 176.5 90.5) (width 0.25) (layer "F.Cu") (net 7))
 (segment (start 71.5 88.346182) (end 71.5 115.25) (width 0.4) (layer "F.Cu") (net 7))
 (segment (start 153.75 63.25) (end 96.596182 63.25) (width 0.4) (layer "F.Cu") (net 7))
 (segment (start 168.25 86.25) (end 168.25 77.75) (width 0.4) (layer "F.Cu") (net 7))
 (segment (start 154.5 111) (end 154.5 127.26) (width 0.25) (layer "F.Cu") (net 18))
 (segment (start 154.5 127.26) (end 156.89 129.65) (width 0.25) (layer "F.Cu") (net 18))
 (segment (start 159 108) (end 156.5 110.5) (width 0.25) (layer "F.Cu") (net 18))
 (segment (start 159 108) (end 173.2 108) (width 0.25) (layer "F.Cu") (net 18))
 (segment (start 155 110.5) (end 154.5 111) (width 0.25) (layer "F.Cu") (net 18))
 (segment (start 156.5 110.5) (end 155 110.5) (width 0.25) (layer "F.Cu") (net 18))
 (segment (start 154.5 110) (end 156 110) (width 0.25) (layer "F.Cu") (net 19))
 (segment (start 154.25 129.5) (end 154.25 129.55) (width 0.4) (layer "F.Cu") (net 19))
 (segment (start 156 110) (end 160 106) (width 0.25) (layer "F.Cu") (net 19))
 (segment (start 173.2 106) (end 160.25 106) (width 0.6) (layer "F.Cu") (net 19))
 (segment (start 154 110.5) (end 154.5 110) (width 0.25) (layer "F.Cu") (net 19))
 (segment (start 154 129.25) (end 154 110.5) (width 0.25) (layer "F.Cu") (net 19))
 (segment (start 161 106) (end 160.25 106) (width 0.25) (layer "F.Cu") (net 19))
 (segment (start 154.25 129.5) (end 154 129.25) (width 0.25) (layer "F.Cu") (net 19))
 (segment (start 154.25 129.55) (end 156.89 132.19) (width 0.4) (layer "F.Cu") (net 19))
 (segment (start 160.15464 106) (end 160.07732 106.07732) (width 0.6) (layer "F.Cu") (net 19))
 (segment (start 160.25 106) (end 160.15464 106) (width 0.6) (layer "F.Cu") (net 19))
 (segment (start 160 106) (end 160.25 106) (width 0.25) (layer "F.Cu") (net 19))
 (segment (start 161.271436 104) (end 155.771436 109.5) (width 0.25) (layer "F.Cu") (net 20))
 (segment (start 155.771436 109.5) (end 154 109.5) (width 0.25) (layer "F.Cu") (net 20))
 (segment (start 173.2 104) (end 161.271436 104) (width 0.25) (layer "F.Cu") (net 20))
 (segment (start 154 109.5) (end 153.5 110) (width 0.25) (layer "F.Cu") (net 20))
 (segment (start 153.5 131.34) (end 156.89 134.73) (width 0.25) (layer "F.Cu") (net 20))
 (segment (start 153.5 110) (end 153.5 131.34) (width 0.25) (layer "F.Cu") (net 20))
 (segment (start 153.27 137.27) (end 156.89 137.27) (width 0.25) (layer "F.Cu") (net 21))
 (segment (start 153 137) (end 153.27 137.27) (width 0.25) (layer "F.Cu") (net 21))
 (segment (start 162.635718 102) (end 173.2 102) (width 0.25) (layer "F.Cu") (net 21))
 (segment (start 155.635718 109) (end 153.5 109) (width 0.25) (layer "F.Cu") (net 21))
 (segment (start 162.635718 102) (end 155.635718 109) (width 0.25) (layer "F.Cu") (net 21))
 (segment (start 153.5 109) (end 153 109.5) (width 0.25) (layer "F.Cu") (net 21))
 (segment (start 153 109.5) (end 153 137) (width 0.25) (layer "F.Cu") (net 21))
 (segment (start 153 108.5) (end 152.5 109) (width 0.25) (layer "F.Cu") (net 22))
 (segment (start 152.5 109) (end 152.5 139.5) (width 0.25) (layer "F.Cu") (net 22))
 (segment (start 155.5 108.5) (end 153 108.5) (width 0.25) (layer "F.Cu") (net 22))
 (segment (start 155.69 139.81) (end 156.89 139.81) (width 0.25) (layer "F.Cu") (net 22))
 (segment (start 164 100) (end 155.5 108.5) (width 0.25) (layer "F.Cu") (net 22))
 (segment (start 173.2 100) (end 164 100) (width 0.25) (layer "F.Cu") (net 22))
 (segment (start 152.5 139.5) (end 153.5 140.5) (width 0.25) (layer "F.Cu") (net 22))
 (segment (start 153.5 140.5) (end 155 140.5) (width 0.25) (layer "F.Cu") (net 22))
 (segment (start 155 140.5) (end 155.69 139.81) (width 0.25) (layer "F.Cu") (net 22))
 (segment (start 152 108.5) (end 152 142) (width 0.25) (layer "F.Cu") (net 23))
 (segment (start 152.35 142.35) (end 156.89 142.35) (width 0.25) (layer "F.Cu") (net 23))
 (segment (start 155.135718 108) (end 152.5 108) (width 0.25) (layer "F.Cu") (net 23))
 (segment (start 165.135718 98) (end 155.135718 108) (width 0.25) (layer "F.Cu") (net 23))
 (segment (start 152 142) (end 152.35 142.35) (width 0.25) (layer "F.Cu") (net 23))
 (segment (start 173.2 98) (end 165.135718 98) (width 0.25) (layer "F.Cu") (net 23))
 (segment (start 152.5 108) (end 152 108.5) (width 0.25) (layer "F.Cu") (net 23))
 (segment (start 155 107.5) (end 152 107.5) (width 0.25) (layer "F.Cu") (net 24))
 (segment (start 173.2 96) (end 166.5 96) (width 0.25) (layer "F.Cu") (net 24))
 (segment (start 152 107.5) (end 151.5 108) (width 0.25) (layer "F.Cu") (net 24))
 (segment (start 151.5 108) (end 151.5 144) (width 0.25) (layer "F.Cu") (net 24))
 (segment (start 151.5 144) (end 152.39 144.89) (width 0.25) (layer "F.Cu") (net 24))
 (segment (start 152.39 144.89) (end 156.89 144.89) (width 0.25) (layer "F.Cu") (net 24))
 (segment (start 166.5 96) (end 155 107.5) (width 0.25) (layer "F.Cu") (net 24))
 (segment (start 97.5 64.25) (end 79 82.75) (width 0.4) (layer "F.Cu") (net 6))
 (segment (start 167.5 86.75) (end 167.5 78.25) (width 0.4) (layer "F.Cu") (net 6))
 (segment (start 79 113) (end 77.25 114.75) (width 0.4) (layer "F.Cu") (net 6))
 (segment (start 173.2 92) (end 172.75 92) (width 0.4) (layer "F.Cu") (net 6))
 (segment (start 172.75 92) (end 167.5 86.75) (width 0.4) (layer "F.Cu") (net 6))
 (segment (start 175.5 92) (end 176 92.5) (width 0.25) (layer "F.Cu") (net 6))
 (segment (start 173.2 92) (end 175.5 92) (width 0.25) (layer "F.Cu") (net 6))
 (segment (start 176 92.5) (end 176 148.64) (width 0.25) (layer "F.Cu") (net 6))
 (segment (start 153.5 64.25) (end 97.5 64.25) (width 0.4) (layer "F.Cu") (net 6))
 (segment (start 79 82.75) (end 79 113) (width 0.4) (layer "F.Cu") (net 6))
 (segment (start 77.25 114.75) (end 74.5 114.75) (width 0.4) (layer "F.Cu") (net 6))
 (segment (start 176 148.64) (end 172.13 152.51) (width 0.25) (layer "F.Cu") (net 6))
 (segment (start 167.5 78.25) (end 153.5 64.25) (width 0.4) (layer "F.Cu") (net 6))
 (segment (start 178.25 136.23) (end 172.13 142.35) (width 0.4) (layer "B.Cu") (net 1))
 (segment (start 178.25 81.25) (end 178.25 136.23) (width 0.4) (layer "B.Cu") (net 1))
 (segment (start 87.25 97.25) (end 122.25 62.25) (width 0.4) (layer "B.Cu") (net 1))
 (segment (start 74.5 97.25) (end 87.25 97.25) (width 0.4) (layer "B.Cu") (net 1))
 (segment (start 159.25 62.25) (end 178.25 81.25) (width 0.4) (layer "B.Cu") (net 1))
 (segment (start 122.25 62.25) (end 159.25 62.25) (width 0.4) (layer "B.Cu") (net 1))
 (segment (start 122.5 63) (end 84.75 100.75) (width 0.4) (layer "B.Cu") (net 2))
 (segment (start 172.13 139.81) (end 173.44 139.81) (width 0.4) (layer "B.Cu") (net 2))
 (segment (start 173.44 139.81) (end 177.5 135.75) (width 0.4) (layer "B.Cu") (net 2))
 (segment (start 158.75 63) (end 122.5 63) (width 0.4) (layer "B.Cu") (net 2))
 (segment (start 177.5 81.75) (end 158.75 63) (width 0.4) (layer "B.Cu") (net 2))
 (segment (start 177.5 135.75) (end 177.5 81.75) (width 0.4) (layer "B.Cu") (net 2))
 (segment (start 84.75 100.75) (end 74.5 100.75) (width 0.4) (layer "B.Cu") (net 2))
 (segment (start 160 132.101278) (end 163.5 135.601278) (width 0.25) (layer "B.Cu") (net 28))
 (segment (start 163.5 149.5) (end 163.97 149.97) (width 0.25) (layer "B.Cu") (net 28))
 (segment (start 163.5 135.601278) (end 163.5 149.5) (width 0.25) (layer "B.Cu") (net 28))
 (segment (start 162.45 90) (end 160 92.45) (width 0.25) (layer "B.Cu") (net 28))
 (segment (start 160 92.45) (end 160 132.101278) (width 0.25) (layer "B.Cu") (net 28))
 (segment (start 163.97 149.97) (end 172.13 149.97) (width 0.25) (layer "B.Cu") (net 28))
 (segment (start 176.75 82) (end 176.75 132.65) (width 0.4) (layer "B.Cu") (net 3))
 (segment (start 83.25 103.25) (end 122.75 63.75) (width 0.4) (layer "B.Cu") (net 3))
 (segment (start 122.75 63.75) (end 158.5 63.75) (width 0.4) (layer "B.Cu") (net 3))
 (segment (start 176.75 132.65) (end 172.13 137.27) (width 0.4) (layer "B.Cu") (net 3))
 (segment (start 158.5 63.75) (end 176.75 82) (width 0.4) (layer "B.Cu") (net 3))
 (segment (start 75.5 103.25) (end 74.5 104.25) (width 0.4) (layer "B.Cu") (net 3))
 (segment (start 83.25 103.25) (end 75.5 103.25) (width 0.4) (layer "B.Cu") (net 3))
 (segment (start 166.23 134.73) (end 172.13 134.73) (width 0.25) (layer "B.Cu") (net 30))
 (segment (start 165 133.5) (end 166.23 134.73) (width 0.25) (layer "B.Cu") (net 30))
 (segment (start 165 98.55) (end 165 133.5) (width 0.25) (layer "B.Cu") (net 30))
 (segment (start 162.45 96) (end 165 98.55) (width 0.25) (layer "B.Cu") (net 30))
 (segment (start 167.19 132.19) (end 172.13 132.19) (width 0.25) (layer "B.Cu") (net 31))
 (segment (start 166.5 98.05) (end 166.5 131.5) (width 0.25) (layer "B.Cu") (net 31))
 (segment (start 166.5 131.5) (end 167.19 132.19) (width 0.25) (layer "B.Cu") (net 31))
 (segment (start 162.45 94) (end 166.5 98.05) (width 0.25) (layer "B.Cu") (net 31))
 (segment (start 175.5 128.25) (end 174.1 129.65) (width 0.4) (layer "B.Cu") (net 4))
 (segment (start 170.25 88) (end 174.75 88) (width 0.4) (layer "B.Cu") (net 4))
 (segment (start 168.25 86) (end 170.25 88) (width 0.4) (layer "B.Cu") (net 4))
 (segment (start 168.25 74.75) (end 168.25 86) (width 0.4) (layer "B.Cu") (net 4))
 (segment (start 175.5 88.75) (end 175.5 128.25) (width 0.4) (layer "B.Cu") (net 4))
 (segment (start 86 101.75) (end 123.25 64.5) (width 0.4) (layer "B.Cu") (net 4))
 (segment (start 123.25 64.5) (end 158 64.5) (width 0.4) (layer "B.Cu") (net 4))
 (segment (start 158 64.5) (end 168.25 74.75) (width 0.4) (layer "B.Cu") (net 4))
 (segment (start 174.1 129.65) (end 172.13 129.65) (width 0.4) (layer "B.Cu") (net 4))
 (segment (start 85.5 107.75) (end 86 107.25) (width 0.4) (layer "B.Cu") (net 4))
 (segment (start 74.5 107.75) (end 85.5 107.75) (width 0.4) (layer "B.Cu") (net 4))
 (segment (start 174.75 88) (end 175.5 88.75) (width 0.4) (layer "B.Cu") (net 4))
 (segment (start 86 107.25) (end 86 101.75) (width 0.4) (layer "B.Cu") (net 4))
 (segment (start 82.25 133.25) (end 82.25 111.5) (width 0.4) (layer "F.Cu") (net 8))
 (segment (start 98.751671 66.65048) (end 142.15048 66.65048) (width 0.4) (layer "F.Cu") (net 8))
 (segment (start 142.15048 66.65048) (end 148.5 73) (width 0.4) (layer "F.Cu") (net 8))
 (segment (start 82.25 111.5) (end 80 109.25) (width 0.4) (layer "F.Cu") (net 8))
 (segment (start 80 109.25) (end 80 85.402151) (width 0.4) (layer "F.Cu") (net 8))
 (segment (start 80 85.402151) (end 98.751671 66.65048) (width 0.4) (layer "F.Cu") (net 8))
 (segment (start 173.5 156.5) (end 177 153) (width 0.4) (layer "B.Cu") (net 8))
 (segment (start 177 153) (end 177 149.76) (width 0.4) (layer "B.Cu") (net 8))
 (segment (start 148.5 73) (end 151 75.5) (width 0.4) (layer "B.Cu") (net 8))
 (segment (start 151 75.5) (end 151 152) (width 0.4) (layer "B.Cu") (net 8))
 (segment (start 151 152) (end 155.5 156.5) (width 0.4) (layer "B.Cu") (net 8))
 (segment (start 155.5 156.5) (end 173.5 156.5) (width 0.4) (layer "B.Cu") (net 8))
 (segment (start 177 149.76) (end 172.13 144.89) (width 0.4) (layer "B.Cu") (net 8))
 (segment (start 97.5 104.5) (end 90.75 111.25) (width 0.4) (layer "B.Cu") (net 5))
 (segment (start 174.75 124.49) (end 174.75 89.5) (width 0.4) (layer "B.Cu") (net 5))
 (segment (start 174 88.75) (end 169.25 88.75) (width 0.4) (layer "B.Cu") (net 5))
 (segment (start 90.75 111.25) (end 74.5 111.25) (width 0.4) (layer "B.Cu") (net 5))
 (segment (start 167.25 75.75) (end 156.75 65.25) (width 0.4) (layer "B.Cu") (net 5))
 (segment (start 123.5 65.25) (end 97.5 91.25) (width 0.4) (layer "B.Cu") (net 5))
 (segment (start 172.13 127.11) (end 174.75 124.49) (width 0.4) (layer "B.Cu") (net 5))
 (segment (start 169.25 88.75) (end 167.25 86.75) (width 0.4) (layer "B.Cu") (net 5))
 (segment (start 167.25 86.75) (end 167.25 75.75) (width 0.4) (layer "B.Cu") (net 5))
 (segment (start 97.5 91.25) (end 97.5 104.5) (width 0.4) (layer "B.Cu") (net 5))
 (segment (start 174.75 89.5) (end 174 88.75) (width 0.4) (layer "B.Cu") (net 5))
 (segment (start 156.75 65.25) (end 123.5 65.25) (width 0.4) (layer "B.Cu") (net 5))
 (segment (start 89 130) (end 85.25 126.25) (width 0.4) (layer "F.Cu") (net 9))
 (segment (start 85.25 126.25) (end 85.25 88.25) (width 0.4) (layer "F.Cu") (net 9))
 (segment (start 85.25 88.25) (end 100.5 73) (width 0.4) (layer "F.Cu") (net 9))
 (segment (start 89 133.25) (end 89 130) (width 0.4) (layer "F.Cu") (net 9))
 (segment (start 103 86) (end 116 86) (width 0.4) (layer "F.Cu") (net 13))
 (segment (start 92 133.25) (end 99 126.25) (width 0.4) (layer "F.Cu") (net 13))
 (segment (start 99 90) (end 103 86) (width 0.4) (layer "F.Cu") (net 13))
 (segment (start 99 126.25) (end 99 90) (width 0.4) (layer "F.Cu") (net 13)))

